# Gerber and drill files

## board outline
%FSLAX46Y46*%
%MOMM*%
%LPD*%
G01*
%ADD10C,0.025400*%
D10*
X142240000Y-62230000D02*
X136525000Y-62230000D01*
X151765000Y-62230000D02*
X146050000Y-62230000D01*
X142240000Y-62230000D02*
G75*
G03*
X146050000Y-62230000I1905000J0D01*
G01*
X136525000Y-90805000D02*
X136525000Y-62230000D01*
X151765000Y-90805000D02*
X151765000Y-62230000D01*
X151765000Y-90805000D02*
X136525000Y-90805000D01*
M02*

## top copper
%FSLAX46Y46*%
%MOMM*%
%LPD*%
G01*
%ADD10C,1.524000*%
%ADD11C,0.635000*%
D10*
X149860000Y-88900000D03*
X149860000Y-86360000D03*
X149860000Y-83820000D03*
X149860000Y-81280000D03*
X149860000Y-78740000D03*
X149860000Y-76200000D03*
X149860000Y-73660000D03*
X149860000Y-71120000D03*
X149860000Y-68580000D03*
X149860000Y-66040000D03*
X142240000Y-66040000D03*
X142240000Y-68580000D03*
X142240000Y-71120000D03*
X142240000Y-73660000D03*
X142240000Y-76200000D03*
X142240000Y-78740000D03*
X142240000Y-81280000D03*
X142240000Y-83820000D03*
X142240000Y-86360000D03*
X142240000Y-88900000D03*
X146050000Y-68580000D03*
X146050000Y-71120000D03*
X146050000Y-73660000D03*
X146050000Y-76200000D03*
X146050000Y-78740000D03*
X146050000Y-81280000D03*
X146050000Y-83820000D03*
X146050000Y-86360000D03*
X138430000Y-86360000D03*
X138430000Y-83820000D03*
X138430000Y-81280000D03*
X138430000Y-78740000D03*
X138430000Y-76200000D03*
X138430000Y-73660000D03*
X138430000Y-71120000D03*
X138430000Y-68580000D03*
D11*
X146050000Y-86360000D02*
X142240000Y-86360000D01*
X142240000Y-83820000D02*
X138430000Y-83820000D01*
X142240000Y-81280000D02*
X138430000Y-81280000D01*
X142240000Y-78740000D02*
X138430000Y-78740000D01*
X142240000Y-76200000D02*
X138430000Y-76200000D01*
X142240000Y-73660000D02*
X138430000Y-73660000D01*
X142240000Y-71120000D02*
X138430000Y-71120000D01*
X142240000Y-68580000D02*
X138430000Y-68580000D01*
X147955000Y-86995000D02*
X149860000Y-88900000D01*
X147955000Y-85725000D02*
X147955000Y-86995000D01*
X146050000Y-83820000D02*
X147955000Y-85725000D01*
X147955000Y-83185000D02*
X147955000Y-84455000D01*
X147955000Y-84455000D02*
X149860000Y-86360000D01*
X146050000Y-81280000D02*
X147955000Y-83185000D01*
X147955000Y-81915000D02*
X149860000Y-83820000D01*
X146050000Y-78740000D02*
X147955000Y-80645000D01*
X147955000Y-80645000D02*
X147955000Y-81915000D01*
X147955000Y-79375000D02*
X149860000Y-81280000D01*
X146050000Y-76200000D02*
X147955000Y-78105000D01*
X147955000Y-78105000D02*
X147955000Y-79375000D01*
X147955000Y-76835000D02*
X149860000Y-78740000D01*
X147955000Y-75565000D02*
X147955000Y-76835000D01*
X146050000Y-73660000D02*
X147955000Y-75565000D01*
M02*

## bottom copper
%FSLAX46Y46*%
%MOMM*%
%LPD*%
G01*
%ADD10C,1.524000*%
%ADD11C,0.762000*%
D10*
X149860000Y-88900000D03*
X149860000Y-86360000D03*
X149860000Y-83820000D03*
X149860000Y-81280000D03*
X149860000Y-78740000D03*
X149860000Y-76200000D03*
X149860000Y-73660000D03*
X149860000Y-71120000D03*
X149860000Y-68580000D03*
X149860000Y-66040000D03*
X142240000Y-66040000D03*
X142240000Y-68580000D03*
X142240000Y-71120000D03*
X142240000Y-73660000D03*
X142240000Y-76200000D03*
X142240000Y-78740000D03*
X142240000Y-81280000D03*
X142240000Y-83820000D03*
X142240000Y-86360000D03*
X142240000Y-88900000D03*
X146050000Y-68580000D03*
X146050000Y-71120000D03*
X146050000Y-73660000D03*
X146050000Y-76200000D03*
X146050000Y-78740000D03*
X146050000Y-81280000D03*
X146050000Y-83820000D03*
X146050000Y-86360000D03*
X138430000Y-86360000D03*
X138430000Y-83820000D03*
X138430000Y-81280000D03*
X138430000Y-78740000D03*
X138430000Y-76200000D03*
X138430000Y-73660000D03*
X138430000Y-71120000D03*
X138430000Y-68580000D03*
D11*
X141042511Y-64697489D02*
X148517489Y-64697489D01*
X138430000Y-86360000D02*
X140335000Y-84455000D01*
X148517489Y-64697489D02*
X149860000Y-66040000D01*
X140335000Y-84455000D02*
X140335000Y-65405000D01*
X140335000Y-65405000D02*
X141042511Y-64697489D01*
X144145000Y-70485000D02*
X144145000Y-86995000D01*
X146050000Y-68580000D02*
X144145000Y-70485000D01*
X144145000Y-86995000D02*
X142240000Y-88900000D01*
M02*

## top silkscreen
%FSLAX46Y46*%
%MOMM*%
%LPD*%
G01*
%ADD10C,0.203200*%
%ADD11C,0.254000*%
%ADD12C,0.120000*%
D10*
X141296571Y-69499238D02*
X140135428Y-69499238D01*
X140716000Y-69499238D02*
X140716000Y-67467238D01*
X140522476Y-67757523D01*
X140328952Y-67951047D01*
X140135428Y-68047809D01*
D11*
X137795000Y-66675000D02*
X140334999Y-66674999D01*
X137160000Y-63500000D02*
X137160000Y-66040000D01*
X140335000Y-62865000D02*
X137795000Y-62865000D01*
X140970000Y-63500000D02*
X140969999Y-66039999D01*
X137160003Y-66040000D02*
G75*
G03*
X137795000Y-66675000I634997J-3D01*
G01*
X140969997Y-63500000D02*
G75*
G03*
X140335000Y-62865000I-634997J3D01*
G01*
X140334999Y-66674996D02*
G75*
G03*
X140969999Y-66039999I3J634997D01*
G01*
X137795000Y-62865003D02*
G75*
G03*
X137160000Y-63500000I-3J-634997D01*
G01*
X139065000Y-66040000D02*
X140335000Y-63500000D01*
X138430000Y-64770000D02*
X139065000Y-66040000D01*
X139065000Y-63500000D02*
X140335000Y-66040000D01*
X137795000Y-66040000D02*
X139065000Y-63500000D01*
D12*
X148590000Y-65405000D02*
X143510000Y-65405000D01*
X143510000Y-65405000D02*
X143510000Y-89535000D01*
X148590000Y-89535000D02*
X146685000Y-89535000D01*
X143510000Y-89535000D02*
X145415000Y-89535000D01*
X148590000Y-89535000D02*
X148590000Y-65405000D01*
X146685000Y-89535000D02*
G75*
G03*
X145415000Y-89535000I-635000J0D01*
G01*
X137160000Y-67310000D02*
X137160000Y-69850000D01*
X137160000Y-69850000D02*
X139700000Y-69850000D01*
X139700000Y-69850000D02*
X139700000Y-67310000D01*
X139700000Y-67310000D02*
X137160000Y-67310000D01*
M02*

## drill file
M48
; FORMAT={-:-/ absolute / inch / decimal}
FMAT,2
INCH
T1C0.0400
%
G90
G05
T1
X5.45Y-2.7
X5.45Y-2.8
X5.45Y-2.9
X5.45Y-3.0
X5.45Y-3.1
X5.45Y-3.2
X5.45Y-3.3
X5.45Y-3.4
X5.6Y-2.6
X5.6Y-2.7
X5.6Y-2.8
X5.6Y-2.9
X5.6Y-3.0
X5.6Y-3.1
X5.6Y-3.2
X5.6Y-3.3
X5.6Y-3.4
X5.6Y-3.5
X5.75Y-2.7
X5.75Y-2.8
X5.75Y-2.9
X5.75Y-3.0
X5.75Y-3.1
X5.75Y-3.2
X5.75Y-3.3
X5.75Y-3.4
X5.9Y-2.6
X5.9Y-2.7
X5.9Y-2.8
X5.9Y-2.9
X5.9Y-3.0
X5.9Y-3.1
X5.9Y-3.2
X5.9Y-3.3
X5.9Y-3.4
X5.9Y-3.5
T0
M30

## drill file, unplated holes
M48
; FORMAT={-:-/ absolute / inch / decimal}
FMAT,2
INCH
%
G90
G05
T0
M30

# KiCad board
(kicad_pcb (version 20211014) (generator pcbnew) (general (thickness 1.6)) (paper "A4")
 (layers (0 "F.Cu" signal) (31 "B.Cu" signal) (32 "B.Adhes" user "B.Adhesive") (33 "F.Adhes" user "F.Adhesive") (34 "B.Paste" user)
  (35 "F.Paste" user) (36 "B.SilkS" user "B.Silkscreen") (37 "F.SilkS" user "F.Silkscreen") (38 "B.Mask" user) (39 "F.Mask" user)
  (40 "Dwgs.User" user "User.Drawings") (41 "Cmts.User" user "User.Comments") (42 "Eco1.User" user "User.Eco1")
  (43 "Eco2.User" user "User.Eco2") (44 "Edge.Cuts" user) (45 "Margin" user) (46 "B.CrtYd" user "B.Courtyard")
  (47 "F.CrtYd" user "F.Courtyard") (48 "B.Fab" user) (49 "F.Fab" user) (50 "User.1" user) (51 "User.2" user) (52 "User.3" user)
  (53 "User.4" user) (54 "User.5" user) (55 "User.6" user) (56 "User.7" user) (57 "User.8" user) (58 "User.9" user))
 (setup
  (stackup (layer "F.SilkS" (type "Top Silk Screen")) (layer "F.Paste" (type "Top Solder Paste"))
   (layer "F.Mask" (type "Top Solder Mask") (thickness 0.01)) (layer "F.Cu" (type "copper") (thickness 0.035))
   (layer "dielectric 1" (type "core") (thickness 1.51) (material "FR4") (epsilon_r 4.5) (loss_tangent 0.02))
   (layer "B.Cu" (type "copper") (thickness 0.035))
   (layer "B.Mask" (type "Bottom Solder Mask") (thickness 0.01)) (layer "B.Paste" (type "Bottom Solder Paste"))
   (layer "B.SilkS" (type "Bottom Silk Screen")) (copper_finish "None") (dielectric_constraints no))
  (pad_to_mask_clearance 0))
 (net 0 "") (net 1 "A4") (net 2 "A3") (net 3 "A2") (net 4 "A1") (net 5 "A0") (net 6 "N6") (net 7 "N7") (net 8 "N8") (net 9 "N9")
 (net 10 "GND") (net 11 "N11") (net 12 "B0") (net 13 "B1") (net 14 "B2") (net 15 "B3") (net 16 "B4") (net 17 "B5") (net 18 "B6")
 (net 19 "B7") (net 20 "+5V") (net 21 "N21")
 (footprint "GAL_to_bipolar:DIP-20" (layer "F.Cu") (at 146.05 77.47 180)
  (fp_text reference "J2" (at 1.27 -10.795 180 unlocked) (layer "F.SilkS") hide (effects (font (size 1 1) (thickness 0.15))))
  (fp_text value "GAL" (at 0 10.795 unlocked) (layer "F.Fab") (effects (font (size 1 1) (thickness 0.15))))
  (fp_line (start -2.54 12.065) (end 2.54 12.065) (layer "F.SilkS") (width 0.12))
  (fp_line (start 2.54 12.065) (end 2.54 -12.065) (layer "F.SilkS") (width 0.12))
  (fp_line (start 2.54 -12.065) (end 0.635 -12.065) (layer "F.SilkS") (width 0.12))
  (fp_line (start -2.54 -12.065) (end -2.54 12.065) (layer "F.SilkS") (width 0.12))
  (fp_line (start -2.54 -12.065) (end -0.635 -12.065) (layer "F.SilkS") (width 0.12))
  (fp_arc (start 0.635 -12.065) (mid 0 -11.43) (end -0.635 -12.065) (layer "F.SilkS") (width 0.12))
  (pad "1" thru_hole circle (at -3.81 -11.43 180) (size 1.524 1.524) (drill 1.016) (layers *.Cu *.Mask) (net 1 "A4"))
  (pad "2" thru_hole circle (at -3.81 -8.89 180) (size 1.524 1.524) (drill 1.016) (layers *.Cu *.Mask) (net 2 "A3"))
  (pad "3" thru_hole circle (at -3.81 -6.35 180) (size 1.524 1.524) (drill 1.016) (layers *.Cu *.Mask) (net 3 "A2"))
  (pad "4" thru_hole circle (at -3.81 -3.81 180) (size 1.524 1.524) (drill 1.016) (layers *.Cu *.Mask) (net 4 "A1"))
  (pad "5" thru_hole circle (at -3.81 -1.27 180) (size 1.524 1.524) (drill 1.016) (layers *.Cu *.Mask) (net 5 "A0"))
  (pad "6" thru_hole circle (at -3.81 1.27 180) (size 1.524 1.524) (drill 1.016) (layers *.Cu *.Mask) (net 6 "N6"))
  (pad "7" thru_hole circle (at -3.81 3.81 180) (size 1.524 1.524) (drill 1.016) (layers *.Cu *.Mask) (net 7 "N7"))
  (pad "8" thru_hole circle (at -3.81 6.35 180) (size 1.524 1.524) (drill 1.016) (layers *.Cu *.Mask) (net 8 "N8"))
  (pad "9" thru_hole circle (at -3.81 8.89 180) (size 1.524 1.524) (drill 1.016) (layers *.Cu *.Mask) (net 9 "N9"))
  (pad "10" thru_hole circle (at -3.81 11.43 180) (size 1.524 1.524) (drill 1.016) (layers *.Cu *.Mask) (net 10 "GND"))
  (pad "11" thru_hole circle (at 3.81 11.43 180) (size 1.524 1.524) (drill 1.016) (layers *.Cu *.Mask) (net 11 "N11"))
  (pad "12" thru_hole circle (at 3.81 8.89 180) (size 1.524 1.524) (drill 1.016) (layers *.Cu *.Mask) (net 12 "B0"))
  (pad "13" thru_hole circle (at 3.81 6.35 180) (size 1.524 1.524) (drill 1.016) (layers *.Cu *.Mask) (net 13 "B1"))
  (pad "14" thru_hole circle (at 3.81 3.81 180) (size 1.524 1.524) (drill 1.016) (layers *.Cu *.Mask) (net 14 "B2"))
  (pad "15" thru_hole circle (at 3.81 1.27 180) (size 1.524 1.524) (drill 1.016) (layers *.Cu *.Mask) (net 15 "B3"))
  (pad "16" thru_hole circle (at 3.81 -1.27 180) (size 1.524 1.524) (drill 1.016) (layers *.Cu *.Mask) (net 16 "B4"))
  (pad "17" thru_hole circle (at 3.81 -3.81 180) (size 1.524 1.524) (drill 1.016) (layers *.Cu *.Mask) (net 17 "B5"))
  (pad "18" thru_hole circle (at 3.81 -6.35 180) (size 1.524 1.524) (drill 1.016) (layers *.Cu *.Mask) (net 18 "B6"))
  (pad "19" thru_hole circle (at 3.81 -8.89 180) (size 1.524 1.524) (drill 1.016) (layers *.Cu *.Mask) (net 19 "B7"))
  (pad "20" thru_hole circle (at 3.81 -11.43 180) (size 1.524 1.524) (drill 1.016) (layers *.Cu *.Mask) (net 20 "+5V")))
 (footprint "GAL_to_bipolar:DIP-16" (layer "F.Cu") (at 142.24 77.47)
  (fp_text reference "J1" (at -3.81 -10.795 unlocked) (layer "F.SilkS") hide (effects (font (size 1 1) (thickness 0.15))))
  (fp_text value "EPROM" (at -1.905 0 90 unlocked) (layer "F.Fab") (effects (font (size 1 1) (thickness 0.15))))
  (fp_line (start -5.08 -10.16) (end -5.08 -7.62) (layer "F.SilkS") (width 0.12))
  (fp_line (start -2.54 -10.16) (end -5.08 -10.16) (layer "F.SilkS") (width 0.12))
  (fp_line (start -5.08 -7.62) (end -2.54 -7.62) (layer "F.SilkS") (width 0.12))
  (fp_line (start -2.54 -7.62) (end -2.54 -10.16) (layer "F.SilkS") (width 0.12))
  (pad "1" thru_hole circle (at -3.81 -8.89) (size 1.524 1.524) (drill 1.016) (layers *.Cu *.Mask) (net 12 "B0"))
  (pad "2" thru_hole circle (at -3.81 -6.35) (size 1.524 1.524) (drill 1.016) (layers *.Cu *.Mask) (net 13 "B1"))
  (pad "3" thru_hole circle (at -3.81 -3.81) (size 1.524 1.524) (drill 1.016) (layers *.Cu *.Mask) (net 14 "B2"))
  (pad "4" thru_hole circle (at -3.81 -1.27) (size 1.524 1.524) (drill 1.016) (layers *.Cu *.Mask) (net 15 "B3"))
  (pad "5" thru_hole circle (at -3.81 1.27) (size 1.524 1.524) (drill 1.016) (layers *.Cu *.Mask) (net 16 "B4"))
  (pad "6" thru_hole circle (at -3.81 3.81) (size 1.524 1.524) (drill 1.016) (layers *.Cu *.Mask) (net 17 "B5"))
  (pad "7" thru_hole circle (at -3.81 6.35) (size 1.524 1.524) (drill 1.016) (layers *.Cu *.Mask) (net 18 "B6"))
  (pad "8" thru_hole circle (at -3.81 8.89) (size 1.524 1.524) (drill 1.016) (layers *.Cu *.Mask) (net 10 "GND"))
  (pad "9" thru_hole circle (at 3.81 8.89) (size 1.524 1.524) (drill 1.016) (layers *.Cu *.Mask) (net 19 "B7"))
  (pad "10" thru_hole circle (at 3.81 6.35) (size 1.524 1.524) (drill 1.016) (layers *.Cu *.Mask) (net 1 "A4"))
  (pad "11" thru_hole circle (at 3.81 3.81) (size 1.524 1.524) (drill 1.016) (layers *.Cu *.Mask) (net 2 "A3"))
  (pad "12" thru_hole circle (at 3.81 1.27) (size 1.524 1.524) (drill 1.016) (layers *.Cu *.Mask) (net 3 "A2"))
  (pad "13" thru_hole circle (at 3.81 -1.27) (size 1.524 1.524) (drill 1.016) (layers *.Cu *.Mask) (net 4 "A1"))
  (pad "14" thru_hole circle (at 3.81 -3.81) (size 1.524 1.524) (drill 1.016) (layers *.Cu *.Mask) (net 5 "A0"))
  (pad "15" thru_hole circle (at 3.81 -6.35) (size 1.524 1.524) (drill 1.016) (layers *.Cu *.Mask) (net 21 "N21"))
  (pad "16" thru_hole circle (at 3.81 -8.89) (size 1.524 1.524) (drill 1.016) (layers *.Cu *.Mask) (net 20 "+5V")))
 (gr_line (start 138.43 64.77) (end 139.065 66.04) (layer "F.SilkS") (width 0.254))
 (gr_line (start 137.16 63.5) (end 137.16 66.04) (layer "F.SilkS") (width 0.254))
 (gr_arc (start 137.16 63.5) (mid 137.345987 63.050988) (end 137.795 62.865) (layer "F.SilkS") (width 0.254))
 (gr_line (start 137.795 66.04) (end 139.065 63.5) (layer "F.SilkS") (width 0.254))
 (gr_line (start 140.335 62.865) (end 137.795 62.865) (layer "F.SilkS") (width 0.254))
 (gr_arc (start 140.335 62.865) (mid 140.784012 63.050987) (end 140.97 63.5) (layer "F.SilkS") (width 0.254))
 (gr_line (start 140.97 63.5) (end 140.969999 66.039999) (layer "F.SilkS") (width 0.254))
 (gr_arc (start 137.795 66.675) (mid 137.345988 66.489013) (end 137.16 66.04) (layer "F.SilkS") (width 0.254))
 (gr_arc (start 140.969999 66.039999) (mid 140.784012 66.489011) (end 140.334999 66.674999) (layer "F.SilkS") (width 0.254))
 (gr_line (start 137.795 66.675) (end 140.334999 66.674999) (layer "F.SilkS") (width 0.254))
 (gr_line (start 139.065 66.04) (end 140.335 63.5) (layer "F.SilkS") (width 0.254))
 (gr_line (start 139.065 63.5) (end 140.335 66.04) (layer "F.SilkS") (width 0.254))
 (gr_line (start 151.765 90.805) (end 136.525 90.805) (layer "Edge.Cuts") (width 0.0254))
 (gr_arc (start 146.05 62.23) (mid 144.145 64.135) (end 142.24 62.23) (layer "Edge.Cuts") (width 0.0254))
 (gr_line (start 151.765 62.23) (end 146.05 62.23) (layer "Edge.Cuts") (width 0.0254))
 (gr_line (start 142.24 62.23) (end 136.525 62.23) (layer "Edge.Cuts") (width 0.0254))
 (gr_line (start 151.765 90.805) (end 151.765 62.23) (layer "Edge.Cuts") (width 0.0254))
 (gr_line (start 136.525 90.805) (end 136.525 62.23) (layer "Edge.Cuts") (width 0.0254))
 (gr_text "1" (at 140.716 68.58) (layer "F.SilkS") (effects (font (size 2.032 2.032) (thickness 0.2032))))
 (segment (start 142.24 68.58) (end 138.43 68.58) (width 0.635) (layer "F.Cu") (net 12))
 (segment (start 142.24 71.12) (end 138.43 71.12) (width 0.635) (layer "F.Cu") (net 13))
 (segment (start 142.24 73.66) (end 138.43 73.66) (width 0.635) (layer "F.Cu") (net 14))
 (segment (start 142.24 76.2) (end 138.43 76.2) (width 0.635) (layer "F.Cu") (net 15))
 (segment (start 142.24 78.74) (end 138.43 78.74) (width 0.635) (layer "F.Cu") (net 16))
 (segment (start 142.24 81.28) (end 138.43 81.28) (width 0.635) (layer "F.Cu") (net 17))
 (segment (start 142.24 83.82) (end 138.43 83.82) (width 0.635) (layer "F.Cu") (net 18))
 (segment (start 141.042511 64.697489) (end 148.517489 64.697489) (width 0.762) (layer "B.Cu") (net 10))
 (segment (start 140.335 84.455) (end 140.335 65.405) (width 0.762) (layer "B.Cu") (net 10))
 (segment (start 140.335 65.405) (end 141.042511 64.697489) (width 0.762) (layer "B.Cu") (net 10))
 (segment (start 138.43 86.36) (end 140.335 84.455) (width 0.762) (layer "B.Cu") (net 10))
 (segment (start 148.517489 64.697489) (end 149.86 66.04) (width 0.762) (layer "B.Cu") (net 10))
 (segment (start 146.05 86.36) (end 142.24 86.36) (width 0.635) (layer "F.Cu") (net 19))
 (segment (start 146.05 83.82) (end 147.955 85.725) (width 0.635) (layer "F.Cu") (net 1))
 (segment (start 147.955 85.725) (end 147.955 86.995) (width 0.635) (layer "F.Cu") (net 1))
 (segment (start 147.955 86.995) (end 149.86 88.9) (width 0.635) (layer "F.Cu") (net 1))
 (segment (start 147.955 84.455) (end 149.86 86.36) (width 0.635) (layer "F.Cu") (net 2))
 (segment (start 146.05 81.28) (end 147.955 83.185) (width 0.635) (layer "F.Cu") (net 2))
 (segment (start 147.955 83.185) (end 147.955 84.455) (width 0.635) (layer "F.Cu") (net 2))
 (segment (start 146.05 78.74) (end 147.955 80.645) (width 0.635) (layer "F.Cu") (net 3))
 (segment (start 147.955 80.645) (end 147.955 81.915) (width 0.635) (layer "F.Cu") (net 3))
 (segment (start 147.955 81.915) (end 149.86 83.82) (width 0.635) (layer "F.Cu") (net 3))
 (segment (start 147.955 78.105) (end 147.955 79.375) (width 0.635) (layer "F.Cu") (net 4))
 (segment (start 147.955 79.375) (end 149.86 81.28) (width 0.635) (layer "F.Cu") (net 4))
 (segment (start 146.05 76.2) (end 147.955 78.105) (width 0.635) (layer "F.Cu") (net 4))
 (segment (start 146.05 73.66) (end 147.955 75.565) (width 0.635) (layer "F.Cu") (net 5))
 (segment (start 147.955 75.565) (end 147.955 76.835) (width 0.635) (layer "F.Cu") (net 5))
 (segment (start 147.955 76.835) (end 149.86 78.74) (width 0.635) (layer "F.Cu") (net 5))
 (segment (start 144.145 86.995) (end 142.24 88.9) (width 0.762) (layer "B.Cu") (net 20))
 (segment (start 146.05 68.58) (end 144.145 70.485) (width 0.762) (layer "B.Cu") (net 20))
 (segment (start 144.145 70.485) (end 144.145 86.995) (width 0.762) (layer "B.Cu") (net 20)))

